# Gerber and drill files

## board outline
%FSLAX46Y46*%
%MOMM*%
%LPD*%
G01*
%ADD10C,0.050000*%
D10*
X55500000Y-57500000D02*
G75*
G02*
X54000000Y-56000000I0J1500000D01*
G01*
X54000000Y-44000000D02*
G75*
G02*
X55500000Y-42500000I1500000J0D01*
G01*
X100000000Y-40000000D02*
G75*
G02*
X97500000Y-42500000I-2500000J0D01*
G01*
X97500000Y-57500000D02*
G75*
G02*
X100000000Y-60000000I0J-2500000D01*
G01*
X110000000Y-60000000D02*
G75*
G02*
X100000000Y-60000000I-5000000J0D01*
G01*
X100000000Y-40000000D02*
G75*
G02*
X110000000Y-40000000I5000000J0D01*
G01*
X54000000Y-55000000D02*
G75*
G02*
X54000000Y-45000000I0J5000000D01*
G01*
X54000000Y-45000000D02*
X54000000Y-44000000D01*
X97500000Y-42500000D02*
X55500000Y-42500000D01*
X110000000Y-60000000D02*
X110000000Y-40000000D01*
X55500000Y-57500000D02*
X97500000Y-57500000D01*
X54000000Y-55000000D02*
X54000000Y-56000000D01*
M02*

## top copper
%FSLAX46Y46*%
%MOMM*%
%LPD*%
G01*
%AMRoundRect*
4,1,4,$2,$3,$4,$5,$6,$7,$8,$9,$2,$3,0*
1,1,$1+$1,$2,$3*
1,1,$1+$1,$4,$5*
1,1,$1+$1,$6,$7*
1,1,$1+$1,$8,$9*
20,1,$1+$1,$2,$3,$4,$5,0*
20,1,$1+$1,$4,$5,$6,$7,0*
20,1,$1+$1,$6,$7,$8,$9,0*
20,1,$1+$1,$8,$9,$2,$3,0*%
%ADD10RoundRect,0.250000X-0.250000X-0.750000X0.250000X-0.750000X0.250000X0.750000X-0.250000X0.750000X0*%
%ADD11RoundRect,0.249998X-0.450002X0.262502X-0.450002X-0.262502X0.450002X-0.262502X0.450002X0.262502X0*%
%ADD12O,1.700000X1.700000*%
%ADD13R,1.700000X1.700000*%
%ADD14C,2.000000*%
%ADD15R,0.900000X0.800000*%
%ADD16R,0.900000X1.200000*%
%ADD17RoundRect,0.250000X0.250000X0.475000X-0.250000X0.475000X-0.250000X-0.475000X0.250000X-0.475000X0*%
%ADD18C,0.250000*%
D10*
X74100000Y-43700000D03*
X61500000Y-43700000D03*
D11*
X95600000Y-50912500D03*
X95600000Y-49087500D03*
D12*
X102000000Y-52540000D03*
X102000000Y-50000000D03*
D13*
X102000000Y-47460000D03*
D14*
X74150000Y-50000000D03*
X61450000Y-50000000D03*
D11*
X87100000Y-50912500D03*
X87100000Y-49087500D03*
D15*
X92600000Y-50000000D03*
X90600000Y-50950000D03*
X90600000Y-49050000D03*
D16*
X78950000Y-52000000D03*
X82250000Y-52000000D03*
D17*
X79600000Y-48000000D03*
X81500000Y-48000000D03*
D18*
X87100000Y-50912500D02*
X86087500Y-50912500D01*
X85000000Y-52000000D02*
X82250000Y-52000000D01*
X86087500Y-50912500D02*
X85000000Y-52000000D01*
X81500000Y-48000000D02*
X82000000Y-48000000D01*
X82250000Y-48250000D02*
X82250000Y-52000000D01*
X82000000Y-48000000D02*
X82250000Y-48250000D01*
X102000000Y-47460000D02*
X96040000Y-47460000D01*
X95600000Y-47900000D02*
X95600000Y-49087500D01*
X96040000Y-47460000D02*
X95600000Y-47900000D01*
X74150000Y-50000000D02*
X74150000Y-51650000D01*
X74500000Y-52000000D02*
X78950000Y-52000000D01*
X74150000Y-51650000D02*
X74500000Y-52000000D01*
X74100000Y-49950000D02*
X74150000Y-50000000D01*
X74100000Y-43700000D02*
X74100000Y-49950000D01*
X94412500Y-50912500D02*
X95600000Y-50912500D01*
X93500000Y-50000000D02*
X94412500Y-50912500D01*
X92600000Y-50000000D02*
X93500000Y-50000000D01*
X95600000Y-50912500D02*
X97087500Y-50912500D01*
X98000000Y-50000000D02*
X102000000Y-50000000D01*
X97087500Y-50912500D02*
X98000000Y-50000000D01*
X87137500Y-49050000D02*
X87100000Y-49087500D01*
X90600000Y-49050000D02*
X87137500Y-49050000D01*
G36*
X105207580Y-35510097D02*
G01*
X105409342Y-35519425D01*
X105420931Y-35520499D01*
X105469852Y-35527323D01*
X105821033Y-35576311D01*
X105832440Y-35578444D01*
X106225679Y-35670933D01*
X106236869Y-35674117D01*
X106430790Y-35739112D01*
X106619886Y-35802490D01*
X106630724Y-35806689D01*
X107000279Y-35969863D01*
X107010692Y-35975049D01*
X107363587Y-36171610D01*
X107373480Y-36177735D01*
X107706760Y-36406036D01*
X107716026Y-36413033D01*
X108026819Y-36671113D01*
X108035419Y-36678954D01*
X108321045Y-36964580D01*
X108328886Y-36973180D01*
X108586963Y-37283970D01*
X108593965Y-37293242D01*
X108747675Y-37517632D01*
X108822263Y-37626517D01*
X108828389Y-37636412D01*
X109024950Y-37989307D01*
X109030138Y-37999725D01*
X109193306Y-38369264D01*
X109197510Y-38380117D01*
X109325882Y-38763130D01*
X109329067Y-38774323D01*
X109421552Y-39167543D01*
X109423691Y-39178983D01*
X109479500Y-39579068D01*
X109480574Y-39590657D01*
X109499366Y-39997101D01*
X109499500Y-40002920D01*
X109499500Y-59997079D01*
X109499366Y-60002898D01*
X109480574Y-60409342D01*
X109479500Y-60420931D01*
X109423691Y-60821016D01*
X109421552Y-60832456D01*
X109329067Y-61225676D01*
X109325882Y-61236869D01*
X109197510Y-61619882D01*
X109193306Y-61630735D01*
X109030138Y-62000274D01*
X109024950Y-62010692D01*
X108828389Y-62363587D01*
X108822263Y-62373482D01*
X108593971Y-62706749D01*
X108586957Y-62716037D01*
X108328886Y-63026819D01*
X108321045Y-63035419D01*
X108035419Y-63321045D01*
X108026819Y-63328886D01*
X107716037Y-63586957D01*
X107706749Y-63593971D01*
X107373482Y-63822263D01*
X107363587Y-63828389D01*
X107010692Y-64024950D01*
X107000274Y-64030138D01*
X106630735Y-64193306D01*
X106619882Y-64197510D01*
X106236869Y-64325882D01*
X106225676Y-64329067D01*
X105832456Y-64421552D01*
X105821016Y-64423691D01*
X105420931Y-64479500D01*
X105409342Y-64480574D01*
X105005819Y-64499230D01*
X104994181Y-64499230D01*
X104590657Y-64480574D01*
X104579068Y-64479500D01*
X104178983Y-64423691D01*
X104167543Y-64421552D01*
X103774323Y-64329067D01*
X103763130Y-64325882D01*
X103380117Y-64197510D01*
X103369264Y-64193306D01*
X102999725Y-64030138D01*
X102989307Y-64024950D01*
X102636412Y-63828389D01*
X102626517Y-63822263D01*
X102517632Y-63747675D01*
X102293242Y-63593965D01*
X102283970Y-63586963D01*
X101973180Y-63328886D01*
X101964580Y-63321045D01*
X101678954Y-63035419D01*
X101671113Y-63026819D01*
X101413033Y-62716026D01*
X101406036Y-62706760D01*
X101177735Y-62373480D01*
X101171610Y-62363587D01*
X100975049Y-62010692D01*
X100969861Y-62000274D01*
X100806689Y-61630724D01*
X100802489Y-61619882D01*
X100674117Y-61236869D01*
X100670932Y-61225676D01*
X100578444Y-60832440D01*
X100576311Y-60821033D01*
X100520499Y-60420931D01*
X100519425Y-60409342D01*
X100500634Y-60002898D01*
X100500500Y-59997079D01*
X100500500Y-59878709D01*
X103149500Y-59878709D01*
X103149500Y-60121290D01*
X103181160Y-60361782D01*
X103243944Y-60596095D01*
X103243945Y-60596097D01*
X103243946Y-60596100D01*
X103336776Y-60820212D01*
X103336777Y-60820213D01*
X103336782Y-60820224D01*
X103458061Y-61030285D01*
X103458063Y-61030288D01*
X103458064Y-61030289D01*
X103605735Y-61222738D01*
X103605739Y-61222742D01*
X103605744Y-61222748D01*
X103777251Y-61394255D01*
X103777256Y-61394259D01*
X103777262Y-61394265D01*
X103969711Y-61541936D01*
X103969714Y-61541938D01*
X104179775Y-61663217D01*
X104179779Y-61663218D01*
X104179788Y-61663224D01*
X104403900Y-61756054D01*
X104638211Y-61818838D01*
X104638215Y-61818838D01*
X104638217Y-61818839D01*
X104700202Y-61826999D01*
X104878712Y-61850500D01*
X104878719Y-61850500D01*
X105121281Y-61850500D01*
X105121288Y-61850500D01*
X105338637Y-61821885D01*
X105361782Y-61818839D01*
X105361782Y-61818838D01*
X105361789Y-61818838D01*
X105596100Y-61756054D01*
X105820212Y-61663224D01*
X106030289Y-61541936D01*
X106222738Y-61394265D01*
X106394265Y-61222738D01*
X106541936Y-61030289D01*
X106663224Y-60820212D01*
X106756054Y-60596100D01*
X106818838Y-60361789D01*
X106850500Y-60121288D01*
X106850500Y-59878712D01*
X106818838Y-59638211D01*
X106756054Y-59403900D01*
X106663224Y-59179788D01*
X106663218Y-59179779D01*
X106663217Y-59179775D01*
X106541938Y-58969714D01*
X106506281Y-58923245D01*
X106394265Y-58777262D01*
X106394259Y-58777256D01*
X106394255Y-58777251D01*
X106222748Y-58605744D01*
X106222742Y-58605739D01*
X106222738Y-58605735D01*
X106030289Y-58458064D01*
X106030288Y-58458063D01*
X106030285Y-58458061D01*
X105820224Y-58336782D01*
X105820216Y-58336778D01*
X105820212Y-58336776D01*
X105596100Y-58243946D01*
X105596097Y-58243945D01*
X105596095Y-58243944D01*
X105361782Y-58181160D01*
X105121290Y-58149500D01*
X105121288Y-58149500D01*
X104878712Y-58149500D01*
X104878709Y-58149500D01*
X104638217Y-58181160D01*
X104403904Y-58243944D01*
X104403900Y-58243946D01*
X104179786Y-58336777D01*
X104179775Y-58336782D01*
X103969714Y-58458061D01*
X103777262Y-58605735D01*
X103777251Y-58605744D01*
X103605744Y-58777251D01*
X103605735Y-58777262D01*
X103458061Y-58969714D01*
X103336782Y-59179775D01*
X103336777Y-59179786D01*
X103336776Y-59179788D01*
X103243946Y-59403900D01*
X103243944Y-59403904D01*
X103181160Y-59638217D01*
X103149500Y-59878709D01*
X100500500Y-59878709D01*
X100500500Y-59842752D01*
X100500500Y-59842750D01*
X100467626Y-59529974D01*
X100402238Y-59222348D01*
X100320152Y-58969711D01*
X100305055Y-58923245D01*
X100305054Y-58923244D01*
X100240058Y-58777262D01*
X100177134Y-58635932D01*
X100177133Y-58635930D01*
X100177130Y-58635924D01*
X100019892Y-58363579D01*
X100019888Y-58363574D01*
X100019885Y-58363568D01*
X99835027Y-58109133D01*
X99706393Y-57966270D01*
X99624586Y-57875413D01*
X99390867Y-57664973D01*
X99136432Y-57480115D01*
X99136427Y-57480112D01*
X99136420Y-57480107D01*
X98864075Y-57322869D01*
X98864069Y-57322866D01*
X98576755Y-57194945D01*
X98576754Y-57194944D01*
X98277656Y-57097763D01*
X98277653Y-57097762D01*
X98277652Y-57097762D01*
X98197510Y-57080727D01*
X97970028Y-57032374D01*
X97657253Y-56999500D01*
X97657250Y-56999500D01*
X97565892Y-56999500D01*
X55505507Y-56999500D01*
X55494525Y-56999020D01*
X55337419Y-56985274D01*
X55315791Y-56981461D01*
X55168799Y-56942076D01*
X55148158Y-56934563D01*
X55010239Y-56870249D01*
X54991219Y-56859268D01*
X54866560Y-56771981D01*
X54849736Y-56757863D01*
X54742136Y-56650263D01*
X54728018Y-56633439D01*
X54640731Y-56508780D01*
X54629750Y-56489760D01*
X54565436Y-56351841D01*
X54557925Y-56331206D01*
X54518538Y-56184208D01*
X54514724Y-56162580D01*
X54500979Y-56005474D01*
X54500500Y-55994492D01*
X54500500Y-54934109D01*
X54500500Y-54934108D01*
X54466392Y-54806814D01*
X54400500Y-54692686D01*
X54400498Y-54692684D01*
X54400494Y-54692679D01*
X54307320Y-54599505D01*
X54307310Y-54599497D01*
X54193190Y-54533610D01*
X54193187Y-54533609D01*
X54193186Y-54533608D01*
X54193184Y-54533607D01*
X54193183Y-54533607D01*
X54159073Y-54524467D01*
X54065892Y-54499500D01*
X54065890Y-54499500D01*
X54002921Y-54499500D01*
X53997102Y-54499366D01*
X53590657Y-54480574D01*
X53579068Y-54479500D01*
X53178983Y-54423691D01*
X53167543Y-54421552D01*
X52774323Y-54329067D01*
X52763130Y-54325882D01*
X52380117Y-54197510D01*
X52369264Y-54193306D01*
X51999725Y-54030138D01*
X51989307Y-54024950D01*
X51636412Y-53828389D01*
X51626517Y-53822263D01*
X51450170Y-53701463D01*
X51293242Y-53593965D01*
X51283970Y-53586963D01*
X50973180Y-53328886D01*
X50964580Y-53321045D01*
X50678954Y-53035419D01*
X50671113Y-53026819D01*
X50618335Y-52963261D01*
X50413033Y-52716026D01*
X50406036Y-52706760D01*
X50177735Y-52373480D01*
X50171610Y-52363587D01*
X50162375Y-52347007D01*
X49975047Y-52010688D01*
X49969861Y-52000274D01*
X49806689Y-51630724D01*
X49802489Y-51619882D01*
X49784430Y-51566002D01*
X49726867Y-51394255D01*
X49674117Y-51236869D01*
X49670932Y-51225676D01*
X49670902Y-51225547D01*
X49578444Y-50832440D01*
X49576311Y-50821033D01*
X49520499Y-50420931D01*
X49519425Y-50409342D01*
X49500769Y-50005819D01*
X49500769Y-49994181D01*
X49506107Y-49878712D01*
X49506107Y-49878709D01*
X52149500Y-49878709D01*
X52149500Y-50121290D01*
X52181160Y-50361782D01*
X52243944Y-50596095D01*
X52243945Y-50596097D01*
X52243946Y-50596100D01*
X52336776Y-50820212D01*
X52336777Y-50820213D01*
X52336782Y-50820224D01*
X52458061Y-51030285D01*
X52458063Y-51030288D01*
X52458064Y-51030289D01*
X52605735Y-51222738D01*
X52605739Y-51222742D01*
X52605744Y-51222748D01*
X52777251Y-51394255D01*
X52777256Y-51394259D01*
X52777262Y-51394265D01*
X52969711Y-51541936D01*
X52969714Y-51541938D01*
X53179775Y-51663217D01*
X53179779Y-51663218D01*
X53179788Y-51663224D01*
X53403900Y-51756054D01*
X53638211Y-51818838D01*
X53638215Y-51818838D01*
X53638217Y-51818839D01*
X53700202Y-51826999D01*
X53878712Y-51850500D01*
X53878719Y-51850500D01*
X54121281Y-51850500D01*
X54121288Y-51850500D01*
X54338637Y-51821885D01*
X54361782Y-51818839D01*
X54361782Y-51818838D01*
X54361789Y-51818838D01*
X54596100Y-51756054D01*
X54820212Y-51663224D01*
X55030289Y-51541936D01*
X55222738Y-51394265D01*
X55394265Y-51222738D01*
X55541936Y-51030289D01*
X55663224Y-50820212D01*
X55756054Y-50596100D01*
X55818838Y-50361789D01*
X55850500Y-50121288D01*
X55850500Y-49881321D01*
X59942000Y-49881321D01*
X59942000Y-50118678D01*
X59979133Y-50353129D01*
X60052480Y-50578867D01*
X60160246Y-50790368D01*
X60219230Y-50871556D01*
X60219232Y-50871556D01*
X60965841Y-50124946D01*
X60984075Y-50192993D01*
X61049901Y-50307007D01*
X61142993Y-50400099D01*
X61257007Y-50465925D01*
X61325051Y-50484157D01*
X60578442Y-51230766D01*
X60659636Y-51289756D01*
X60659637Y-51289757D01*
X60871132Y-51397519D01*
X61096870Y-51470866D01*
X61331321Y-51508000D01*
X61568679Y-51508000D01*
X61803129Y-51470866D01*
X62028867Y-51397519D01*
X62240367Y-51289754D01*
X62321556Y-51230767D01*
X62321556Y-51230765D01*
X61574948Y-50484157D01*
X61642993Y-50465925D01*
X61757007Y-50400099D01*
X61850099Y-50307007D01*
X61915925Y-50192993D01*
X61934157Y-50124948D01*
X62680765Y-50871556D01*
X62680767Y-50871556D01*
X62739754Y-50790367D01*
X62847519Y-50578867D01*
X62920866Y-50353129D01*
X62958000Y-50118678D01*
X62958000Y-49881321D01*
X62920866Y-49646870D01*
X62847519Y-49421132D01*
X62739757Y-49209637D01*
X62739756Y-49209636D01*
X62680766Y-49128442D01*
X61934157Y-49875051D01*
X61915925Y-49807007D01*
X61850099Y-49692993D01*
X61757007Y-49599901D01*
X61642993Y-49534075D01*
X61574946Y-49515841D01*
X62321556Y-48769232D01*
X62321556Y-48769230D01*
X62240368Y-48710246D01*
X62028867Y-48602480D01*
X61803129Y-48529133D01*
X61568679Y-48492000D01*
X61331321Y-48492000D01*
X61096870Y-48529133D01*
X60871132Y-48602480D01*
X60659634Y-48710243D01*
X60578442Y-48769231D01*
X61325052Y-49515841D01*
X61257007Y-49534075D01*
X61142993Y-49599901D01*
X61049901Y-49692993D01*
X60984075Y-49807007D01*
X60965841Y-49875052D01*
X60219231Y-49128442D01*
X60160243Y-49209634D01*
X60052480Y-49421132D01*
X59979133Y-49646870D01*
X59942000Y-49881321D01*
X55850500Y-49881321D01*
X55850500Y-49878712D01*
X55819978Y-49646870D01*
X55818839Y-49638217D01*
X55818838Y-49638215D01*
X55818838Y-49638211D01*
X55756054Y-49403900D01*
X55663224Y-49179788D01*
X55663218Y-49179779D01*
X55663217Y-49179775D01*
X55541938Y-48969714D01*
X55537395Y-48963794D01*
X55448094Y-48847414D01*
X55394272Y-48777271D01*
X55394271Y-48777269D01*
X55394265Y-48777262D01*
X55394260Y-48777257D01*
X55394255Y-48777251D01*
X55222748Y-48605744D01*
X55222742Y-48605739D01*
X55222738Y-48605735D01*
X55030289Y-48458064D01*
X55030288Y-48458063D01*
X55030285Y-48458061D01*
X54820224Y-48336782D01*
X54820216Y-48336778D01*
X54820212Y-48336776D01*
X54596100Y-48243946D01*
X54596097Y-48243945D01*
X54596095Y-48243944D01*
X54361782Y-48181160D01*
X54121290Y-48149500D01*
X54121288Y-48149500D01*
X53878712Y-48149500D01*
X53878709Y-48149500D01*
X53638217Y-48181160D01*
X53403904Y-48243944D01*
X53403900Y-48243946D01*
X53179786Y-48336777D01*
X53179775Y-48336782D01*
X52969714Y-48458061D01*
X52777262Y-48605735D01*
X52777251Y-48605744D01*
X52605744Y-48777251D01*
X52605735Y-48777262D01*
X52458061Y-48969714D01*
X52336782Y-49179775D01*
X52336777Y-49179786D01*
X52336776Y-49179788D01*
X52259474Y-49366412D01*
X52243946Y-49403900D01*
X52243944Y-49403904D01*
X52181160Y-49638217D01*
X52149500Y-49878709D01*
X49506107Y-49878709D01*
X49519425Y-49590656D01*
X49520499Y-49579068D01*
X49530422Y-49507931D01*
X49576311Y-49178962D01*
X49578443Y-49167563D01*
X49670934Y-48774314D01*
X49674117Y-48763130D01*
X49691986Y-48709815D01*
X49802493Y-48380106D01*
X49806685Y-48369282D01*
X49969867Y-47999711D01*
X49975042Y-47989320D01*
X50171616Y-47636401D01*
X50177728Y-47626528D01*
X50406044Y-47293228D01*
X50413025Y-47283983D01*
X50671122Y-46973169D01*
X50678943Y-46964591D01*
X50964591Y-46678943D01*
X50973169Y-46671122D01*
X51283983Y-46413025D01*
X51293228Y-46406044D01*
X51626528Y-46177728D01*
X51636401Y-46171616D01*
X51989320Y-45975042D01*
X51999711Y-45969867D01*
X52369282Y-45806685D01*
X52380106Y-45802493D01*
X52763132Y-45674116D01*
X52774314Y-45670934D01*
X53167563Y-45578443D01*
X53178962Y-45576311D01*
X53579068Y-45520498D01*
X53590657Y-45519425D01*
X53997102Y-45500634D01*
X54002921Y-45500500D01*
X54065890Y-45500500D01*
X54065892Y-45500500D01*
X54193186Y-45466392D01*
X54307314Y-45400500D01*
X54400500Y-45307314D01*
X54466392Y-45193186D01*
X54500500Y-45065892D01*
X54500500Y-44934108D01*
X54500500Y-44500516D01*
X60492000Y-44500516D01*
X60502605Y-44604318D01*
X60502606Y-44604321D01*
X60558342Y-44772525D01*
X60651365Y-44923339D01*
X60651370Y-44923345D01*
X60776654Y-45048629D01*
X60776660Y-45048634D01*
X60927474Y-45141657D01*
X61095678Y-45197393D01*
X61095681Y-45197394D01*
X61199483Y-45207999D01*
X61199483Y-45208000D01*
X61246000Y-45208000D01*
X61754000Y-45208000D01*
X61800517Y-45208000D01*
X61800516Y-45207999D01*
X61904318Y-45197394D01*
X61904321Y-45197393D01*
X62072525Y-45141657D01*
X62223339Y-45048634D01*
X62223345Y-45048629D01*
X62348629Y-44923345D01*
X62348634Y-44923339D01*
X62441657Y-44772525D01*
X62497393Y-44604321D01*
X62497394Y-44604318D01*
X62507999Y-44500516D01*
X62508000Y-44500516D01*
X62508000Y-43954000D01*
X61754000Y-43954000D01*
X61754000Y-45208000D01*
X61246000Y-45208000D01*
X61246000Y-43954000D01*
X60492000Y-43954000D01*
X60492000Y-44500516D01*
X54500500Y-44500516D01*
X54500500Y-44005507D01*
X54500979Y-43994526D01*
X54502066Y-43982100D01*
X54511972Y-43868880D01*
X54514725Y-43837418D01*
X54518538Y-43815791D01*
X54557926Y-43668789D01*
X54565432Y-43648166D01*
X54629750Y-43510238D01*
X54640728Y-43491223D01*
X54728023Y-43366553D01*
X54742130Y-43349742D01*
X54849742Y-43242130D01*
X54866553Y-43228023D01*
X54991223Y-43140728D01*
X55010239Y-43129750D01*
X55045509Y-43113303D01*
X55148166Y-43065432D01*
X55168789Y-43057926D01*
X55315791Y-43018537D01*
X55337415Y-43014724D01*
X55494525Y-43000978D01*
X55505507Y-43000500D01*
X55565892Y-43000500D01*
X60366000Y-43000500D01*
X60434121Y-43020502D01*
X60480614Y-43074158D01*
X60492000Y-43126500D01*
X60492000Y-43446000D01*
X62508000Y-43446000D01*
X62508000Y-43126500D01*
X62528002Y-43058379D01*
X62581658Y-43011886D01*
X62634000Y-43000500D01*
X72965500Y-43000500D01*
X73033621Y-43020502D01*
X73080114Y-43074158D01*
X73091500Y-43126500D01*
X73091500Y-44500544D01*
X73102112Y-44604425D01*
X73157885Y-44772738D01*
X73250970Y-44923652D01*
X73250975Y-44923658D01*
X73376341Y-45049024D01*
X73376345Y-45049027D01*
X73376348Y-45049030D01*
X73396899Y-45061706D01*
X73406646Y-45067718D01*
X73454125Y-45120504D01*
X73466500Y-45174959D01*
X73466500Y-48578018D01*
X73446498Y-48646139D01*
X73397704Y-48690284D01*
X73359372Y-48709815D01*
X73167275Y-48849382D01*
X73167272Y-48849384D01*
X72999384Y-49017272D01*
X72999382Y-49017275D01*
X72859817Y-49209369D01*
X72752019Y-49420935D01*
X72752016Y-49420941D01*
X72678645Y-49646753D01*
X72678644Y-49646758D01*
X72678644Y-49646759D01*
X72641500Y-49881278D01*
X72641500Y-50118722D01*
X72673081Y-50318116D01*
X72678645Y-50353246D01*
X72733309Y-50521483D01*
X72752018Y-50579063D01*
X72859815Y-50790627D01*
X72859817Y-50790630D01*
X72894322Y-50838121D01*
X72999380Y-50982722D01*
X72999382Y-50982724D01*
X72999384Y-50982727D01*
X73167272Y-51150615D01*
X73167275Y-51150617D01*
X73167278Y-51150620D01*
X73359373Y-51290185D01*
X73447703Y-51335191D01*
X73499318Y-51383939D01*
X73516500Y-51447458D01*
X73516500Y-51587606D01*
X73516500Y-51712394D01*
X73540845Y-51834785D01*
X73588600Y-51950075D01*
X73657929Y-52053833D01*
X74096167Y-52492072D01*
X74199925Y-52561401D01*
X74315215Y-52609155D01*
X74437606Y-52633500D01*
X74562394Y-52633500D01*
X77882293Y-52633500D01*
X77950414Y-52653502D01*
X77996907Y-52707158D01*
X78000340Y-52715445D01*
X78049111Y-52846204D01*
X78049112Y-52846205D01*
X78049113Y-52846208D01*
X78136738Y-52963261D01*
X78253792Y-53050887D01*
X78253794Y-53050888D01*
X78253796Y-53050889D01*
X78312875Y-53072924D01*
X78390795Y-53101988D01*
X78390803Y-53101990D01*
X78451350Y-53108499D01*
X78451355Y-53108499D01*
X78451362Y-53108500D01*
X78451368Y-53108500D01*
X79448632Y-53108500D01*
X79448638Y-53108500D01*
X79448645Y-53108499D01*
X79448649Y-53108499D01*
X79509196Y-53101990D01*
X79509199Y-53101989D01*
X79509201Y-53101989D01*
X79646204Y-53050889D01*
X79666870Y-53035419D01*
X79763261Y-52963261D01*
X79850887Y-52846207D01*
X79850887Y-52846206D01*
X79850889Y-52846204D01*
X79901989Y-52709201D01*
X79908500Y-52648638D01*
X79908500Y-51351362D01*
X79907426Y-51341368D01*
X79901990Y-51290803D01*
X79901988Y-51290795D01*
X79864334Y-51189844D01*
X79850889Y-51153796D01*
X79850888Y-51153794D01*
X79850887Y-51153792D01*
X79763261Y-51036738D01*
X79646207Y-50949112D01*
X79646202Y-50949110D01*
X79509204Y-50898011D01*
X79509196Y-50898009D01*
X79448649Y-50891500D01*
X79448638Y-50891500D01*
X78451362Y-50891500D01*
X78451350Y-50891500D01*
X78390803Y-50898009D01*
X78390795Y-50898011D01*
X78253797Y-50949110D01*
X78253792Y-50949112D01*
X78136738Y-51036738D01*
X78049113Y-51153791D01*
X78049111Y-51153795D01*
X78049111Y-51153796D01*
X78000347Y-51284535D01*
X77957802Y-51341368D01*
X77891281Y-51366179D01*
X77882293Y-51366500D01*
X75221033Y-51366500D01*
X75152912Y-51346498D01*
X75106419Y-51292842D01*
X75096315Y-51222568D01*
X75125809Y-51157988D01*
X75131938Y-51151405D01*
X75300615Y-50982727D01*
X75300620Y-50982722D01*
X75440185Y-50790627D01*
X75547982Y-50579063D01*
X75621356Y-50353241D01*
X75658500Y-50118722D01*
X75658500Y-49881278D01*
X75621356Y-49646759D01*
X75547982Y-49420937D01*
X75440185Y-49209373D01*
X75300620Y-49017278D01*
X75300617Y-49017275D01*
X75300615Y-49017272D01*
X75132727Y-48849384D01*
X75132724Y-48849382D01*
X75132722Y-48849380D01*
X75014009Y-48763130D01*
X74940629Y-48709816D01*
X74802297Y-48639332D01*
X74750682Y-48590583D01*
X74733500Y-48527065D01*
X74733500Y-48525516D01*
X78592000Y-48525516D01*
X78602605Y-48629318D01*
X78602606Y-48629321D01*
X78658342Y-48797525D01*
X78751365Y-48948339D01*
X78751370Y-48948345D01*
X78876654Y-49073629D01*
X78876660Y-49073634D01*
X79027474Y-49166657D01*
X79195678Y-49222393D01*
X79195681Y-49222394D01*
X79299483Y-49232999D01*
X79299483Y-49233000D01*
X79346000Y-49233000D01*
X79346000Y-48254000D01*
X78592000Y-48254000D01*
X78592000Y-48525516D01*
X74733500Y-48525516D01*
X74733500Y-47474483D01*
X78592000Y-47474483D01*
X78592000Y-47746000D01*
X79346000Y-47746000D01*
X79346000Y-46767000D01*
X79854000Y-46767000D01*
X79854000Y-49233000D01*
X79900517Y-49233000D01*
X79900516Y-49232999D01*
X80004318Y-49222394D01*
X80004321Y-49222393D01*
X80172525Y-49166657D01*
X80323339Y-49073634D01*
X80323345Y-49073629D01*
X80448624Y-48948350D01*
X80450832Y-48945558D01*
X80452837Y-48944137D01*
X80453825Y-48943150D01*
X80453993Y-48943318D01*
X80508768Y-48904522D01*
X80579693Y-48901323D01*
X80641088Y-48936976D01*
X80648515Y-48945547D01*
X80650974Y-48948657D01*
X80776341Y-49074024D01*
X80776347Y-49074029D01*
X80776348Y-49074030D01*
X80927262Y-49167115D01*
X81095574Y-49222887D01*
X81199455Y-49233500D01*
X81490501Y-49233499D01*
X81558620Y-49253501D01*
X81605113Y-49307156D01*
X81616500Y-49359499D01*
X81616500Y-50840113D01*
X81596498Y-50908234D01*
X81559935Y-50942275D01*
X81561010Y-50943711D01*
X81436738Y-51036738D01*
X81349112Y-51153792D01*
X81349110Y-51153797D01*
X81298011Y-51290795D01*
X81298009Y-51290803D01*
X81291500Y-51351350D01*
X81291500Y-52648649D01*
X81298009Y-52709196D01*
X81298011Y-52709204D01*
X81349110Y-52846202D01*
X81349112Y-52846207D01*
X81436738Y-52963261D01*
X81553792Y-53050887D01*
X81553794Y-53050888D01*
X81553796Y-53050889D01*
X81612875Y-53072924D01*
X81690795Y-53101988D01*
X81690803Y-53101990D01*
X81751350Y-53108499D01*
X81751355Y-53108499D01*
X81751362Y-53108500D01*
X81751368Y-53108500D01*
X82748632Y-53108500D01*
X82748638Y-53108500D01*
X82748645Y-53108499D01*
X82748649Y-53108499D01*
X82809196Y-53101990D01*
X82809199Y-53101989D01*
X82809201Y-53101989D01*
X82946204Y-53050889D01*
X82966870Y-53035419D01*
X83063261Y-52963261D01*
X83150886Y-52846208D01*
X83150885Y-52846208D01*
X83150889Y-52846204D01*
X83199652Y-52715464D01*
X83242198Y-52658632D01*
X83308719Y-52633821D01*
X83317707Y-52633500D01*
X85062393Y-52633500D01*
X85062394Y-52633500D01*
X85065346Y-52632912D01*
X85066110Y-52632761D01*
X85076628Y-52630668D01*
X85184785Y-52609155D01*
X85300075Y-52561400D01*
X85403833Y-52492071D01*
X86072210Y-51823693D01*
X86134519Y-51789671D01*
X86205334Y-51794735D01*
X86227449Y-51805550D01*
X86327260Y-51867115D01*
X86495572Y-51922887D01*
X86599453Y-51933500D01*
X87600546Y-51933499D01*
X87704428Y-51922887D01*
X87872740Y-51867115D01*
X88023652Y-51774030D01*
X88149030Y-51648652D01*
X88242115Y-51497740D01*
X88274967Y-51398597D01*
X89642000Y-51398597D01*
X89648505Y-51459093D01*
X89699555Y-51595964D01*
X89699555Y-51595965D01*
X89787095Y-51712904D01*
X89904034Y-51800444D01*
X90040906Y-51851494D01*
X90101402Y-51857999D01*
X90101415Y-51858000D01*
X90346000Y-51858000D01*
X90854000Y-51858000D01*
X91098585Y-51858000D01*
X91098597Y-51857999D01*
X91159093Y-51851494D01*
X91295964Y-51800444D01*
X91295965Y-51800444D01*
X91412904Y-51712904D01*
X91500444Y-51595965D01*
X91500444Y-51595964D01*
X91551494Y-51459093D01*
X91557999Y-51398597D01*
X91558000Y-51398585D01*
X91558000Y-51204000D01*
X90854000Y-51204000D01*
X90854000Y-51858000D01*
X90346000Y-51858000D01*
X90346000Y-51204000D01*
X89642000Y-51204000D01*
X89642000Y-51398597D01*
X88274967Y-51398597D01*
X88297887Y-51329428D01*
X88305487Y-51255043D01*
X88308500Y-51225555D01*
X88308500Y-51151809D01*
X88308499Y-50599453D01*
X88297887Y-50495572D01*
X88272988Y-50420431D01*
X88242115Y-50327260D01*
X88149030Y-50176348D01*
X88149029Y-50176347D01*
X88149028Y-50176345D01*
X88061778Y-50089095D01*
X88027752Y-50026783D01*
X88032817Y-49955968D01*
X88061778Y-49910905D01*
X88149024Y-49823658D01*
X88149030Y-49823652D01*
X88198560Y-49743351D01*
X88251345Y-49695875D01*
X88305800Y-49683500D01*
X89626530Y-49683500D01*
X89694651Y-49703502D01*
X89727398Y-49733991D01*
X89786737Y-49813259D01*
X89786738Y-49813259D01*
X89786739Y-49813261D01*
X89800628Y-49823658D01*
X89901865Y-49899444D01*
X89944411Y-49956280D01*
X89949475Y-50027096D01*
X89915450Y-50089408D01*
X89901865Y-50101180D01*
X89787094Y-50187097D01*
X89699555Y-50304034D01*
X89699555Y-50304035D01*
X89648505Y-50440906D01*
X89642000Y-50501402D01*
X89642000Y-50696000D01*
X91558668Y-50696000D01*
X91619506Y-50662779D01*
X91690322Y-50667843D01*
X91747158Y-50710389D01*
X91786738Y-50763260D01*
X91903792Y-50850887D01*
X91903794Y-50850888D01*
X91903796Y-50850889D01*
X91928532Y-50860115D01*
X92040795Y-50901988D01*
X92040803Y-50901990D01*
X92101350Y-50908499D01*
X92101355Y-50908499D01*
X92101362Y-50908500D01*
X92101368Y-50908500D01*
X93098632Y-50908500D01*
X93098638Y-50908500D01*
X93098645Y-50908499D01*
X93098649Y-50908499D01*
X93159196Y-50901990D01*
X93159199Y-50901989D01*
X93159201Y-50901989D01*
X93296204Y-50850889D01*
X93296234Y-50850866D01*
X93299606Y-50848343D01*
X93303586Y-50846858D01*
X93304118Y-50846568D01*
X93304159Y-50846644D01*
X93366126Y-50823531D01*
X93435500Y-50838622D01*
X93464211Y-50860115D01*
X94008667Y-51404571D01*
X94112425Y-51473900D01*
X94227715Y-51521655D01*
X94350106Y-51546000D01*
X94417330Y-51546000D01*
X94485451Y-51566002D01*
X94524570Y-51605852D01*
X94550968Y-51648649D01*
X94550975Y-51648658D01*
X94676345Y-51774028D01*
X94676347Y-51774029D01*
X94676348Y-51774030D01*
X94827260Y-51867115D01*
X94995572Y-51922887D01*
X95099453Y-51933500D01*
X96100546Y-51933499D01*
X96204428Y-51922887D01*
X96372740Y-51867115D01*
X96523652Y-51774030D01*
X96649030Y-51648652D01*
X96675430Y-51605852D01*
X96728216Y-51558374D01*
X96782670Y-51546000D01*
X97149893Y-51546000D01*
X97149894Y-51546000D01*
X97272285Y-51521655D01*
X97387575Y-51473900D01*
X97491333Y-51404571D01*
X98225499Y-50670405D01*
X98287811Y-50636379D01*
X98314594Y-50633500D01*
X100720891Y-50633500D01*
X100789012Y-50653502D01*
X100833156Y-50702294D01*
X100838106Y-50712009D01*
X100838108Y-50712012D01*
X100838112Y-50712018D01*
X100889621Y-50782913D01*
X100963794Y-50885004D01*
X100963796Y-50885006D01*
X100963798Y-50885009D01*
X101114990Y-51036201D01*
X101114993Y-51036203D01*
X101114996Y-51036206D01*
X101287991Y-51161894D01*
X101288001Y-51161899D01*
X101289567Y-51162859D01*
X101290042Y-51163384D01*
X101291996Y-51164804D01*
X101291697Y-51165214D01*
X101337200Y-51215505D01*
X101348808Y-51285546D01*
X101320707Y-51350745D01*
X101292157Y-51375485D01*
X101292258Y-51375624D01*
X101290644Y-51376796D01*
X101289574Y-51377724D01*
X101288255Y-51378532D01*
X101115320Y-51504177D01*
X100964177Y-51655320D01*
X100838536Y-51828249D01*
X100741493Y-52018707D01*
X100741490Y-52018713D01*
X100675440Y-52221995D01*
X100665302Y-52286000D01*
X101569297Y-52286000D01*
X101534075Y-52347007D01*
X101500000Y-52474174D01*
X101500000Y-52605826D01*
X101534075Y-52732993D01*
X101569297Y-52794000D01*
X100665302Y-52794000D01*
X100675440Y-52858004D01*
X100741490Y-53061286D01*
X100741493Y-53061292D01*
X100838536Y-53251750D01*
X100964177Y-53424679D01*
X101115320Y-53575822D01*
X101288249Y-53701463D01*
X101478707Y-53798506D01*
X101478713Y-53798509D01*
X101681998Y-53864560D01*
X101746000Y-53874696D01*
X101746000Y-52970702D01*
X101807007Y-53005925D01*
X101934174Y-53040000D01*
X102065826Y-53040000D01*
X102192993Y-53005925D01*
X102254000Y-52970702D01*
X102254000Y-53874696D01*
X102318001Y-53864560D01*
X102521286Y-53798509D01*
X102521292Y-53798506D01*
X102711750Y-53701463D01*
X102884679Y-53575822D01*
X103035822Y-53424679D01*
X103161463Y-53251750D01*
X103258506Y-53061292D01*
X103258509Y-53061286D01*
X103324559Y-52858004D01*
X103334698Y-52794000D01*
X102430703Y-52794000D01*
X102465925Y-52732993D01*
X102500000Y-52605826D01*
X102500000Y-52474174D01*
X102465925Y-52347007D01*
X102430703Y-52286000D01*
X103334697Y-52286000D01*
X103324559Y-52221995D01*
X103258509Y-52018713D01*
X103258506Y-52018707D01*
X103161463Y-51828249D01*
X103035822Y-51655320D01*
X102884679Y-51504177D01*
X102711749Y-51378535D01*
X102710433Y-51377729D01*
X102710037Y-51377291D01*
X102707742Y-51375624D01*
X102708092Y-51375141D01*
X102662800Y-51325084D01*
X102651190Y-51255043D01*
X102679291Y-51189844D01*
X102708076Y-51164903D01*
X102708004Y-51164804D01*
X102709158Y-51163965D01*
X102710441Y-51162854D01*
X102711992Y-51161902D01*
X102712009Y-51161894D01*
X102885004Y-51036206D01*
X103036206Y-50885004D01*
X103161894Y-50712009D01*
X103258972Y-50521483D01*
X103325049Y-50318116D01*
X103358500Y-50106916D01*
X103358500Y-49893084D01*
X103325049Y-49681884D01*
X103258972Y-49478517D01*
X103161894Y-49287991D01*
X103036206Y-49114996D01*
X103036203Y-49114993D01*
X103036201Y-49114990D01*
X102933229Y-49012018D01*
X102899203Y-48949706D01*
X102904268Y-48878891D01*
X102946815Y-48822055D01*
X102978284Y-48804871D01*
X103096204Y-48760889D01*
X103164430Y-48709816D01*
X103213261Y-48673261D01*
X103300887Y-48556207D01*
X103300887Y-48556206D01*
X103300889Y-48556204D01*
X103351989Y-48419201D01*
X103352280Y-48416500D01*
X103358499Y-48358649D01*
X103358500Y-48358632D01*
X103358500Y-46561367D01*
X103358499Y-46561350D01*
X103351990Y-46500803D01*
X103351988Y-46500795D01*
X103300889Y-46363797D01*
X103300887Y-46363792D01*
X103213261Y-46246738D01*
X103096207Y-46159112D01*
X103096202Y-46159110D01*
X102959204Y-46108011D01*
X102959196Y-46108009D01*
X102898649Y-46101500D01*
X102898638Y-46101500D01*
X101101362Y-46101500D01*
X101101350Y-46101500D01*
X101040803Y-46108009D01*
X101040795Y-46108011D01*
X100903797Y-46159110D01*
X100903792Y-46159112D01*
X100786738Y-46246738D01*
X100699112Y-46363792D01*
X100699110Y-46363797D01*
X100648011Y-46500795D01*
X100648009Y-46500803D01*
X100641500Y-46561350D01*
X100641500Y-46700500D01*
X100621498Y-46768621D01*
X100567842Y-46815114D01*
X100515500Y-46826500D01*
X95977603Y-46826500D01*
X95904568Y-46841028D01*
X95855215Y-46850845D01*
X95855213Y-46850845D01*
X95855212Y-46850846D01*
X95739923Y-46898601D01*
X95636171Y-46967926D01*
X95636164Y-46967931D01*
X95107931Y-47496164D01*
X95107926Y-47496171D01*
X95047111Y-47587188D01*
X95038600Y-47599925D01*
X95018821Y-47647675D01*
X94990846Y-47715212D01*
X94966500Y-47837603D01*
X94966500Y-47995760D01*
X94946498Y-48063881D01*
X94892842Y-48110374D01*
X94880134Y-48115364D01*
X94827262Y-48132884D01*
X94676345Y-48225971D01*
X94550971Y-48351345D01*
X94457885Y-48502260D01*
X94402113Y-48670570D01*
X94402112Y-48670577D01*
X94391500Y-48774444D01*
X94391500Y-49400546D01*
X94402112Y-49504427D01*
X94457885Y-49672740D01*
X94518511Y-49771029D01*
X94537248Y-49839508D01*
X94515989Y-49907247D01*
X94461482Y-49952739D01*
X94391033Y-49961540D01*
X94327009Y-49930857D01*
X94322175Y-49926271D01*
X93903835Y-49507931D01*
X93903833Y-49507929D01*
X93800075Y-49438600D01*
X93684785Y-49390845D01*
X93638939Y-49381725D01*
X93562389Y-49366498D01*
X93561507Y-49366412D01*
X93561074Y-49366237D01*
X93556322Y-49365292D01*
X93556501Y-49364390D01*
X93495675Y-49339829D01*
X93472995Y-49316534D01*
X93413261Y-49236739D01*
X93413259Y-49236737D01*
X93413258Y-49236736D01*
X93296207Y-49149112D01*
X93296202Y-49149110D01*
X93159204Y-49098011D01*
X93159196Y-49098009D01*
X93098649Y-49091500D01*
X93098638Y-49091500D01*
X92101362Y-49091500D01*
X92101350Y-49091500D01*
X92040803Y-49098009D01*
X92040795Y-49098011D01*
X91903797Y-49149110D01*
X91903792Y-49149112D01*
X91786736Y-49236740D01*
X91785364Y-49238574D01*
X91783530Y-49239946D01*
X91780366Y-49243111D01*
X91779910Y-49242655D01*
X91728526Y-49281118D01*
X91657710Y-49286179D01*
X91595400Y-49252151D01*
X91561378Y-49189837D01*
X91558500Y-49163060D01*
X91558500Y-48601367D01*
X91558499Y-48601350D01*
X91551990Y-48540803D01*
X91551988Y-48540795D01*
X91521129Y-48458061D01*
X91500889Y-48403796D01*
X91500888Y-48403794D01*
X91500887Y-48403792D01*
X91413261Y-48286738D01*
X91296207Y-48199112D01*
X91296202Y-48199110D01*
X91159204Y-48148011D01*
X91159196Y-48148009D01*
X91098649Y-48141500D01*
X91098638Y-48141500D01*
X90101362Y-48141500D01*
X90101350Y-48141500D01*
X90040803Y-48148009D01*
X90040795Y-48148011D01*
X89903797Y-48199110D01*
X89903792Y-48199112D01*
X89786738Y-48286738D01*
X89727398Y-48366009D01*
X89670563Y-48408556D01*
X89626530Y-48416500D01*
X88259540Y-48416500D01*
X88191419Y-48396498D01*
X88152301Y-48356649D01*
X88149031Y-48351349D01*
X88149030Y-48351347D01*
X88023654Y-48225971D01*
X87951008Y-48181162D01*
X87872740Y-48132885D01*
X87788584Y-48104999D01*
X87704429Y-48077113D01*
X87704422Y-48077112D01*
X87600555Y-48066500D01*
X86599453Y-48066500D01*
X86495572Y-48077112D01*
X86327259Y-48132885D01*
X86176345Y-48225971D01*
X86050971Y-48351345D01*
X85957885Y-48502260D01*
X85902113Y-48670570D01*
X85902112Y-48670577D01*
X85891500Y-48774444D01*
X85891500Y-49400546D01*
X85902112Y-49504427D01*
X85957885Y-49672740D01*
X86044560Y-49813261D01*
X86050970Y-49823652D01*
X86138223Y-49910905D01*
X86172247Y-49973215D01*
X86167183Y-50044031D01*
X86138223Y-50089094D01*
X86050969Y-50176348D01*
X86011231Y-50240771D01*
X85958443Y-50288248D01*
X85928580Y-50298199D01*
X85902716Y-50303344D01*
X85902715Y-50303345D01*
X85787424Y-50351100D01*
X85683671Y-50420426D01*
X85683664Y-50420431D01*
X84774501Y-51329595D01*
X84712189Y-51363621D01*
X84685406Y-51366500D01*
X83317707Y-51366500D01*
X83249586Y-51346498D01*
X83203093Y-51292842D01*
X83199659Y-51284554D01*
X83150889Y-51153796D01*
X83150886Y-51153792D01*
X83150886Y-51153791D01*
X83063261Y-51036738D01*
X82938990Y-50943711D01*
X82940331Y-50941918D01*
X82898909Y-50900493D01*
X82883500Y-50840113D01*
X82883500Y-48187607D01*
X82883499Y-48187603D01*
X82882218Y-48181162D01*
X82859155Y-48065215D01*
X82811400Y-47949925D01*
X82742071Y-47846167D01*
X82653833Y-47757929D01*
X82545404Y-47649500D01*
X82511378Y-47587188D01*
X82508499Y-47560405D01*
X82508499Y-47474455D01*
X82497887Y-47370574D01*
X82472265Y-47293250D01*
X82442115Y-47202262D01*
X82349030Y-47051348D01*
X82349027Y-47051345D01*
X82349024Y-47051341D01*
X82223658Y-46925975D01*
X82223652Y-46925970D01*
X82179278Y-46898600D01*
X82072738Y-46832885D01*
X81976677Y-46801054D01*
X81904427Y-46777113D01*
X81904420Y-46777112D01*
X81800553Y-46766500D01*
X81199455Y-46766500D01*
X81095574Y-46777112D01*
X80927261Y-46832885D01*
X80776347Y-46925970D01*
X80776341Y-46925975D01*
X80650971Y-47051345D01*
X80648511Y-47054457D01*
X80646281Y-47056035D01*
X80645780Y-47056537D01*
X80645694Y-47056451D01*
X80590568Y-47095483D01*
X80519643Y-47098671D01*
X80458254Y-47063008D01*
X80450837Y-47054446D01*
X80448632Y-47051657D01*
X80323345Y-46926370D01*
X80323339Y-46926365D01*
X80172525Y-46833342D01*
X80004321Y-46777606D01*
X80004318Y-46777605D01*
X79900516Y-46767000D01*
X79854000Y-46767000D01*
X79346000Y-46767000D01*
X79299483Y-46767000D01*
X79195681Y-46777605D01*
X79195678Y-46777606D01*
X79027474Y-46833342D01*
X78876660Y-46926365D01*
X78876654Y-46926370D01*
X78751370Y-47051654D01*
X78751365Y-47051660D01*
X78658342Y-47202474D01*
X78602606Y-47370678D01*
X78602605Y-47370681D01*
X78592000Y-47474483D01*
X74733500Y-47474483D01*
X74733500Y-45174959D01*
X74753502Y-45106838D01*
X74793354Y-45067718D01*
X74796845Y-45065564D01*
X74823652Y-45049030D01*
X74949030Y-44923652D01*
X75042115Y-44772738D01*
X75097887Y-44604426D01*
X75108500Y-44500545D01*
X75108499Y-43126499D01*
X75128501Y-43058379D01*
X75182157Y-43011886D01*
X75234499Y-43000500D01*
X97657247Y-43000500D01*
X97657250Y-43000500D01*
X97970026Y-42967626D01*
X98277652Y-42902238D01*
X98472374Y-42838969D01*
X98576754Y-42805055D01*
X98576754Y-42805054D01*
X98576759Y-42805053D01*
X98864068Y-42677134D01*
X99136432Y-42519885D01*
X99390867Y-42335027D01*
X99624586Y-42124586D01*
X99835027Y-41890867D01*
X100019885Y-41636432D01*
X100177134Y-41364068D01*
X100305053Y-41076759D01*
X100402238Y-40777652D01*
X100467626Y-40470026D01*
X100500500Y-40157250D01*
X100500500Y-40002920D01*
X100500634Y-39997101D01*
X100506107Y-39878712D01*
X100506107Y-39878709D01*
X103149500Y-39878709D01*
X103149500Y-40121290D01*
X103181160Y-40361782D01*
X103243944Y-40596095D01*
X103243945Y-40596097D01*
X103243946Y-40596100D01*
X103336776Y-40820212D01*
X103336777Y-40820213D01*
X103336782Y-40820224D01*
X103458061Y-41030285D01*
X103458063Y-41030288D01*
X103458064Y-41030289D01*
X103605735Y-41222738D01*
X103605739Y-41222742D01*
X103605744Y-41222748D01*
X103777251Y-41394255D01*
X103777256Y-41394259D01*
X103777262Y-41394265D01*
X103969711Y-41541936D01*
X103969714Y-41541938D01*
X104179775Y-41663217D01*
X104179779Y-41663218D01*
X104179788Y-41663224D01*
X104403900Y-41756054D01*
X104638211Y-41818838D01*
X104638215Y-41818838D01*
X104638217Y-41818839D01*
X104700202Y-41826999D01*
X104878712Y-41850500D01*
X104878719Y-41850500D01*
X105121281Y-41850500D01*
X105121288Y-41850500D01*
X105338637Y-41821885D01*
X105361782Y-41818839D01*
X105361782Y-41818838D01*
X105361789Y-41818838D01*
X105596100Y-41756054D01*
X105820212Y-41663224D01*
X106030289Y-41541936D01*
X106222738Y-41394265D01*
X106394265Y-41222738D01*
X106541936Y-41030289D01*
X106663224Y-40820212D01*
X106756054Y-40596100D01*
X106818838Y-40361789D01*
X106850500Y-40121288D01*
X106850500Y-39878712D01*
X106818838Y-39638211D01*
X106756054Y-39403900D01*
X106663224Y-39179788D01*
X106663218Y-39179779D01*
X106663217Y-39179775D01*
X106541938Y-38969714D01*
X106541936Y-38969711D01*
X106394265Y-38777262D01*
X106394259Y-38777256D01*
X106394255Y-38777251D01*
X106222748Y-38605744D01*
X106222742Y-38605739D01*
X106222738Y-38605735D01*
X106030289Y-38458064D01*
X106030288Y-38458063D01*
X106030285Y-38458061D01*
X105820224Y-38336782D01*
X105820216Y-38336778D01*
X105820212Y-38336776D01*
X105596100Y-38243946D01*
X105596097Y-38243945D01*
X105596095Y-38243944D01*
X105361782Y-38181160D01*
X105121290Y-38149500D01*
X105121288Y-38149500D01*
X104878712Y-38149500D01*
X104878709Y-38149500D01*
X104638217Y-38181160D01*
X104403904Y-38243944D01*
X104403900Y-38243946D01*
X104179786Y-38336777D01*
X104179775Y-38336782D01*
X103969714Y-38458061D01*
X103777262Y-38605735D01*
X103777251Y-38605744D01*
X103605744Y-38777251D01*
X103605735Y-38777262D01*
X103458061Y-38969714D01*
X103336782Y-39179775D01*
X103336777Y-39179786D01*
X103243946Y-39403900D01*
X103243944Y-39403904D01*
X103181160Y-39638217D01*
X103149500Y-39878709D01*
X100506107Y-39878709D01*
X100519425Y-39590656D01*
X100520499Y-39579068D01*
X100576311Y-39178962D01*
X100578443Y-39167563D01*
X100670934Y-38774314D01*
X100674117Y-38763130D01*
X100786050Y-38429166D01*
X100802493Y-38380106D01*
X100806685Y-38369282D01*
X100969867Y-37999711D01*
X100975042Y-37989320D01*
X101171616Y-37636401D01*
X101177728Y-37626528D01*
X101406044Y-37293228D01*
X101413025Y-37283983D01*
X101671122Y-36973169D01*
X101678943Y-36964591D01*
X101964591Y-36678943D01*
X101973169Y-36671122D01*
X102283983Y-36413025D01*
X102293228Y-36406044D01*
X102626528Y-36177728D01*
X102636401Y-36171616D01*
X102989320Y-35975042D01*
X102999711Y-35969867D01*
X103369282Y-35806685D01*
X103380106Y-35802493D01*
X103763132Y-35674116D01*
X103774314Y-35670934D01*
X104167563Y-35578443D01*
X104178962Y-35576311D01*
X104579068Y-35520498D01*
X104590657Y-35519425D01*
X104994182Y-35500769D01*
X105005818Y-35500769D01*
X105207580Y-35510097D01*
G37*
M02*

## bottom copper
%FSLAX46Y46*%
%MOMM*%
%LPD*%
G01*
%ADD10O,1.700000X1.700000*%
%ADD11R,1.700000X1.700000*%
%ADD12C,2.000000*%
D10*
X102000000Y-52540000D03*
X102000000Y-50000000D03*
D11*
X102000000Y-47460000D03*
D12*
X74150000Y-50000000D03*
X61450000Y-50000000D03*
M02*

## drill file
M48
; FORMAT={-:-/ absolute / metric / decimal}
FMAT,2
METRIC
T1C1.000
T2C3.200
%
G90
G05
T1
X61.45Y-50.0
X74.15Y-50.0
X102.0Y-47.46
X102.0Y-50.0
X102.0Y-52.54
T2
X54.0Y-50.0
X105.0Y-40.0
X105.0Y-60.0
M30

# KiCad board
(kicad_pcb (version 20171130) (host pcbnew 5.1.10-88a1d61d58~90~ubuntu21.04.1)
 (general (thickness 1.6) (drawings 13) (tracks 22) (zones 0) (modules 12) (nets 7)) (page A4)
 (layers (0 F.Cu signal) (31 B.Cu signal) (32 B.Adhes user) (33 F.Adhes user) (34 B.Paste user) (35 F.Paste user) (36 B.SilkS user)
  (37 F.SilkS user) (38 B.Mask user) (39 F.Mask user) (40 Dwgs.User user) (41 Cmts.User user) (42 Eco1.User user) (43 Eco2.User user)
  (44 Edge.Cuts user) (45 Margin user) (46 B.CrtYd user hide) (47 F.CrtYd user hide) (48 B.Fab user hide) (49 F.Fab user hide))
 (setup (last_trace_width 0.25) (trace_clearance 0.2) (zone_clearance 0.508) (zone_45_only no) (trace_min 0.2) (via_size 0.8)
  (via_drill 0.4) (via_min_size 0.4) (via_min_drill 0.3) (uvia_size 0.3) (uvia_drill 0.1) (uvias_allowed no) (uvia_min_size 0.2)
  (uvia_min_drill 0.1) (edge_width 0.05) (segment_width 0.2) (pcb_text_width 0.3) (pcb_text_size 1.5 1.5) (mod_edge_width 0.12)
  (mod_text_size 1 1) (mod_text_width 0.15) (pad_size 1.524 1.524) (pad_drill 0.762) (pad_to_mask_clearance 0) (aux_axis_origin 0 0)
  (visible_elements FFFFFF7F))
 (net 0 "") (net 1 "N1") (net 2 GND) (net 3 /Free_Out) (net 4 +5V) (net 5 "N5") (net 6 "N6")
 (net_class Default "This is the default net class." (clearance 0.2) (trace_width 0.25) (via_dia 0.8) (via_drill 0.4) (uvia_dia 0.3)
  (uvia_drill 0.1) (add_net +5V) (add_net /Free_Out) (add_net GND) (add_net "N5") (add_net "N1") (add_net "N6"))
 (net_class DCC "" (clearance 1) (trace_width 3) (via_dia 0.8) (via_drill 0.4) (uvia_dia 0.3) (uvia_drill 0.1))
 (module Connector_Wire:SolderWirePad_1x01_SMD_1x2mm (layer F.Cu) (at 74.1 43.7)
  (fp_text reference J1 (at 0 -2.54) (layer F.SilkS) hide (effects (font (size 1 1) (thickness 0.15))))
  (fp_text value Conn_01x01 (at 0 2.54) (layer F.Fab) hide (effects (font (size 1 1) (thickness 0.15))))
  (pad 1 smd roundrect (at 0 0) (size 1 2) (layers F.Cu F.Paste F.Mask) (roundrect_rratio 0.25) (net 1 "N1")))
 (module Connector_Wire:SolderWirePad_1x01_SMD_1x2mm (layer F.Cu) (at 61.5 43.7)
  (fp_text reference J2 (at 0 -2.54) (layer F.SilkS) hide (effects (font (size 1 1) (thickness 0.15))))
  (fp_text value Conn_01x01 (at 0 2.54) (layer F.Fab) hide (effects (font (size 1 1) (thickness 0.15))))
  (pad 1 smd roundrect (at 0 0) (size 1 2) (layers F.Cu F.Paste F.Mask) (roundrect_rratio 0.25) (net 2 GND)))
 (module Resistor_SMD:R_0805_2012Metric (layer F.Cu) (at 95.6 50 270)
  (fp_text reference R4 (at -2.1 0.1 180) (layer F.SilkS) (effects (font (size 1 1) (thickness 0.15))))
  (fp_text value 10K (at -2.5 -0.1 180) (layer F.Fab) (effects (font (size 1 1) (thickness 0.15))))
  (pad 2 smd roundrect (at 0.9125 0 270) (size 1.025 1.4) (layers F.Cu F.Paste F.Mask) (roundrect_rratio 0.2439004878048781)
   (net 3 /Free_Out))
  (pad 1 smd roundrect (at -0.9125 0 270) (size 1.025 1.4) (layers F.Cu F.Paste F.Mask) (roundrect_rratio 0.2439004878048781) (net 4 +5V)))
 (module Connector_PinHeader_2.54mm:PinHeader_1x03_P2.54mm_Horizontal (layer F.Cu) (at 102 47.46)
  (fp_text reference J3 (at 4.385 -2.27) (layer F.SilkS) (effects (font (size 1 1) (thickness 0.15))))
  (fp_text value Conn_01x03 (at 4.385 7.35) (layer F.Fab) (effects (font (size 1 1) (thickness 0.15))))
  (pad 3 thru_hole oval (at 0 5.08) (size 1.7 1.7) (drill 1) (layers *.Cu *.Mask) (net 2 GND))
  (pad 2 thru_hole oval (at 0 2.54) (size 1.7 1.7) (drill 1) (layers *.Cu *.Mask) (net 3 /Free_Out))
  (pad 1 thru_hole rect (at 0 0) (size 1.7 1.7) (drill 1) (layers *.Cu *.Mask) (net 4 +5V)))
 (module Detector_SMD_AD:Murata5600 (layer F.Cu) (at 67.8 50)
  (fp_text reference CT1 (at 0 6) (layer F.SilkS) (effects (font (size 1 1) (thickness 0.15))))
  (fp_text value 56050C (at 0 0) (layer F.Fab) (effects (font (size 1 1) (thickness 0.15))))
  (pad 2 thru_hole circle (at 6.35 0) (size 2 2) (drill 1) (layers *.Cu *.Mask) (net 1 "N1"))
  (pad 1 thru_hole circle (at -6.35 0) (size 2 2) (drill 1) (layers *.Cu *.Mask) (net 2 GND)))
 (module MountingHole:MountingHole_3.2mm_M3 (layer F.Cu) (at 105 60)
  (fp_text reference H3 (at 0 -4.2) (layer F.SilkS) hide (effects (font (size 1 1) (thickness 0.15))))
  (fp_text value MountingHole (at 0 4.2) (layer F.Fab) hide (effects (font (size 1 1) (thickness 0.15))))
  (pad 1 np_thru_hole circle (at 0 0) (size 3.2 3.2) (drill 3.2) (layers *.Cu *.Mask)))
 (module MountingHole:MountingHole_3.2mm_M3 (layer F.Cu) (at 105 40)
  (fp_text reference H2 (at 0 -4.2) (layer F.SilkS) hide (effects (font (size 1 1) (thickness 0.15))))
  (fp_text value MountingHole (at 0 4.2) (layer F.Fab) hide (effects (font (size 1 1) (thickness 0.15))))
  (pad 1 np_thru_hole circle (at 0 0) (size 3.2 3.2) (drill 3.2) (layers *.Cu *.Mask)))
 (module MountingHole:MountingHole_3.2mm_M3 (layer F.Cu) (at 54 50)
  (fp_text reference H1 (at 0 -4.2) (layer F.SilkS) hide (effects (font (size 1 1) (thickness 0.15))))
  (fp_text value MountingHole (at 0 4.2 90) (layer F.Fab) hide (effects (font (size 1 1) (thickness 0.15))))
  (pad 1 np_thru_hole circle (at 0 0) (size 3.2 3.2) (drill 3.2) (layers *.Cu *.Mask)))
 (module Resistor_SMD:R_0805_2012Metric (layer F.Cu) (at 87.1 50 270)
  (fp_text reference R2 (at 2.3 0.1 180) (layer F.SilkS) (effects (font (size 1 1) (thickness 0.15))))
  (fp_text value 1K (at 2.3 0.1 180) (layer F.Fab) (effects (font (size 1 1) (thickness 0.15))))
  (pad 2 smd roundrect (at 0.9125 0 270) (size 1.025 1.4) (layers F.Cu F.Paste F.Mask) (roundrect_rratio 0.2439004878048781) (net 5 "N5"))
  (pad 1 smd roundrect (at -0.9125 0 270) (size 1.025 1.4) (layers F.Cu F.Paste F.Mask) (roundrect_rratio 0.2439004878048781) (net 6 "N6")))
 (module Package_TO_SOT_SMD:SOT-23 (layer F.Cu) (at 91.6 50)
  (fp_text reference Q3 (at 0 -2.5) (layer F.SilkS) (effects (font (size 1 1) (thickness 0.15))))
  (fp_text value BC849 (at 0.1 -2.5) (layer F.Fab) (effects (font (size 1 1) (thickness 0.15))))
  (pad 3 smd rect (at 1 0) (size 0.9 0.8) (layers F.Cu F.Paste F.Mask) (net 3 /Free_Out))
  (pad 2 smd rect (at -1 0.95) (size 0.9 0.8) (layers F.Cu F.Paste F.Mask) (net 2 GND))
  (pad 1 smd rect (at -1 -0.95) (size 0.9 0.8) (layers F.Cu F.Paste F.Mask) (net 6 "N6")))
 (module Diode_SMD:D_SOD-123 (layer F.Cu) (at 80.6 52 180)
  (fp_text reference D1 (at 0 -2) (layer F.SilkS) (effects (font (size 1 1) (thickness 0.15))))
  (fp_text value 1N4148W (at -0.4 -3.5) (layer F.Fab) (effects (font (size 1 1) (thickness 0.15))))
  (pad 2 smd rect (at 1.65 0 180) (size 0.9 1.2) (layers F.Cu F.Paste F.Mask) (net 1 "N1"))
  (pad 1 smd rect (at -1.65 0 180) (size 0.9 1.2) (layers F.Cu F.Paste F.Mask) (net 5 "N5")))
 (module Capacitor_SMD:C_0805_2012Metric (layer F.Cu) (at 80.55 48 180)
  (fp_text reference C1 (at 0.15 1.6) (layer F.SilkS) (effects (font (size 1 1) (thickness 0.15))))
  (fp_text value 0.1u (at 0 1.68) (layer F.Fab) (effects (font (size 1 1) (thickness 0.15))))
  (pad 2 smd roundrect (at 0.95 0 180) (size 1 1.45) (layers F.Cu F.Paste F.Mask) (roundrect_rratio 0.25) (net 2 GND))
  (pad 1 smd roundrect (at -0.95 0 180) (size 1 1.45) (layers F.Cu F.Paste F.Mask) (roundrect_rratio 0.25) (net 5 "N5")))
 (gr_arc (start 55.5 56) (end 54 56) (angle -90) (layer Edge.Cuts) (width 0.05))
 (gr_arc (start 55.5 44) (end 55.5 42.5) (angle -90) (layer Edge.Cuts) (width 0.05))
 (gr_arc (start 97.5 40) (end 97.5 42.5) (angle -90) (layer Edge.Cuts) (width 0.05))
 (gr_arc (start 97.5 60) (end 100 60) (angle -90) (layer Edge.Cuts) (width 0.05))
 (gr_arc (start 105 60) (end 100 60) (angle -180) (layer Edge.Cuts) (width 0.05))
 (gr_arc (start 105 40) (end 110 40) (angle -180) (layer Edge.Cuts) (width 0.05))
 (gr_arc (start 54 50) (end 54 45) (angle -180) (layer Edge.Cuts) (width 0.05))
 (gr_line (start 54 45) (end 54 44) (layer Edge.Cuts) (width 0.05))
 (gr_line (start 97.5 42.5) (end 55.5 42.5) (layer Edge.Cuts) (width 0.05))
 (gr_line (start 110 60) (end 110 40) (layer Edge.Cuts) (width 0.05))
 (gr_line (start 55.5 57.5) (end 97.5 57.5) (layer Edge.Cuts) (width 0.05))
 (gr_line (start 54 55) (end 54 56) (layer Edge.Cuts) (width 0.05))
 (segment (start 87.1 50.9125) (end 86.0875 50.9125) (width 0.25) (layer F.Cu) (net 5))
 (segment (start 85 52) (end 82.25 52) (width 0.25) (layer F.Cu) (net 5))
 (segment (start 86.0875 50.9125) (end 85 52) (width 0.25) (layer F.Cu) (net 5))
 (segment (start 81.5 48) (end 82 48) (width 0.25) (layer F.Cu) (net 5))
 (segment (start 82.25 48.25) (end 82.25 52) (width 0.25) (layer F.Cu) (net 5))
 (segment (start 82 48) (end 82.25 48.25) (width 0.25) (layer F.Cu) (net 5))
 (segment (start 102 47.46) (end 96.04 47.46) (width 0.25) (layer F.Cu) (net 4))
 (segment (start 95.6 47.9) (end 95.6 49.0875) (width 0.25) (layer F.Cu) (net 4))
 (segment (start 96.04 47.46) (end 95.6 47.9) (width 0.25) (layer F.Cu) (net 4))
 (segment (start 74.15 50) (end 74.15 51.65) (width 0.25) (layer F.Cu) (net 1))
 (segment (start 74.5 52) (end 78.95 52) (width 0.25) (layer F.Cu) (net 1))
 (segment (start 74.15 51.65) (end 74.5 52) (width 0.25) (layer F.Cu) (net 1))
 (segment (start 74.1 49.95) (end 74.15 50) (width 0.25) (layer F.Cu) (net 1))
 (segment (start 74.1 43.7) (end 74.1 49.95) (width 0.25) (layer F.Cu) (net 1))
 (segment (start 94.4125 50.9125) (end 95.6 50.9125) (width 0.25) (layer F.Cu) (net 3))
 (segment (start 93.5 50) (end 94.4125 50.9125) (width 0.25) (layer F.Cu) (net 3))
 (segment (start 92.6 50) (end 93.5 50) (width 0.25) (layer F.Cu) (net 3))
 (segment (start 95.6 50.9125) (end 97.0875 50.9125) (width 0.25) (layer F.Cu) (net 3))
 (segment (start 98 50) (end 102 50) (width 0.25) (layer F.Cu) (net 3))
 (segment (start 97.0875 50.9125) (end 98 50) (width 0.25) (layer F.Cu) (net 3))
 (segment (start 87.1375 49.05) (end 87.1 49.0875) (width 0.25) (layer F.Cu) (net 6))
 (segment (start 90.6 49.05) (end 87.1375 49.05) (width 0.25) (layer F.Cu) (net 6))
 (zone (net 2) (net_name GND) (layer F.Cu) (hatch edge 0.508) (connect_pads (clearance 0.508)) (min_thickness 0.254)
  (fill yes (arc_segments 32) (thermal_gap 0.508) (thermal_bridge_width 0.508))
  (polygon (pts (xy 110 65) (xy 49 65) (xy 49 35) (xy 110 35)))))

